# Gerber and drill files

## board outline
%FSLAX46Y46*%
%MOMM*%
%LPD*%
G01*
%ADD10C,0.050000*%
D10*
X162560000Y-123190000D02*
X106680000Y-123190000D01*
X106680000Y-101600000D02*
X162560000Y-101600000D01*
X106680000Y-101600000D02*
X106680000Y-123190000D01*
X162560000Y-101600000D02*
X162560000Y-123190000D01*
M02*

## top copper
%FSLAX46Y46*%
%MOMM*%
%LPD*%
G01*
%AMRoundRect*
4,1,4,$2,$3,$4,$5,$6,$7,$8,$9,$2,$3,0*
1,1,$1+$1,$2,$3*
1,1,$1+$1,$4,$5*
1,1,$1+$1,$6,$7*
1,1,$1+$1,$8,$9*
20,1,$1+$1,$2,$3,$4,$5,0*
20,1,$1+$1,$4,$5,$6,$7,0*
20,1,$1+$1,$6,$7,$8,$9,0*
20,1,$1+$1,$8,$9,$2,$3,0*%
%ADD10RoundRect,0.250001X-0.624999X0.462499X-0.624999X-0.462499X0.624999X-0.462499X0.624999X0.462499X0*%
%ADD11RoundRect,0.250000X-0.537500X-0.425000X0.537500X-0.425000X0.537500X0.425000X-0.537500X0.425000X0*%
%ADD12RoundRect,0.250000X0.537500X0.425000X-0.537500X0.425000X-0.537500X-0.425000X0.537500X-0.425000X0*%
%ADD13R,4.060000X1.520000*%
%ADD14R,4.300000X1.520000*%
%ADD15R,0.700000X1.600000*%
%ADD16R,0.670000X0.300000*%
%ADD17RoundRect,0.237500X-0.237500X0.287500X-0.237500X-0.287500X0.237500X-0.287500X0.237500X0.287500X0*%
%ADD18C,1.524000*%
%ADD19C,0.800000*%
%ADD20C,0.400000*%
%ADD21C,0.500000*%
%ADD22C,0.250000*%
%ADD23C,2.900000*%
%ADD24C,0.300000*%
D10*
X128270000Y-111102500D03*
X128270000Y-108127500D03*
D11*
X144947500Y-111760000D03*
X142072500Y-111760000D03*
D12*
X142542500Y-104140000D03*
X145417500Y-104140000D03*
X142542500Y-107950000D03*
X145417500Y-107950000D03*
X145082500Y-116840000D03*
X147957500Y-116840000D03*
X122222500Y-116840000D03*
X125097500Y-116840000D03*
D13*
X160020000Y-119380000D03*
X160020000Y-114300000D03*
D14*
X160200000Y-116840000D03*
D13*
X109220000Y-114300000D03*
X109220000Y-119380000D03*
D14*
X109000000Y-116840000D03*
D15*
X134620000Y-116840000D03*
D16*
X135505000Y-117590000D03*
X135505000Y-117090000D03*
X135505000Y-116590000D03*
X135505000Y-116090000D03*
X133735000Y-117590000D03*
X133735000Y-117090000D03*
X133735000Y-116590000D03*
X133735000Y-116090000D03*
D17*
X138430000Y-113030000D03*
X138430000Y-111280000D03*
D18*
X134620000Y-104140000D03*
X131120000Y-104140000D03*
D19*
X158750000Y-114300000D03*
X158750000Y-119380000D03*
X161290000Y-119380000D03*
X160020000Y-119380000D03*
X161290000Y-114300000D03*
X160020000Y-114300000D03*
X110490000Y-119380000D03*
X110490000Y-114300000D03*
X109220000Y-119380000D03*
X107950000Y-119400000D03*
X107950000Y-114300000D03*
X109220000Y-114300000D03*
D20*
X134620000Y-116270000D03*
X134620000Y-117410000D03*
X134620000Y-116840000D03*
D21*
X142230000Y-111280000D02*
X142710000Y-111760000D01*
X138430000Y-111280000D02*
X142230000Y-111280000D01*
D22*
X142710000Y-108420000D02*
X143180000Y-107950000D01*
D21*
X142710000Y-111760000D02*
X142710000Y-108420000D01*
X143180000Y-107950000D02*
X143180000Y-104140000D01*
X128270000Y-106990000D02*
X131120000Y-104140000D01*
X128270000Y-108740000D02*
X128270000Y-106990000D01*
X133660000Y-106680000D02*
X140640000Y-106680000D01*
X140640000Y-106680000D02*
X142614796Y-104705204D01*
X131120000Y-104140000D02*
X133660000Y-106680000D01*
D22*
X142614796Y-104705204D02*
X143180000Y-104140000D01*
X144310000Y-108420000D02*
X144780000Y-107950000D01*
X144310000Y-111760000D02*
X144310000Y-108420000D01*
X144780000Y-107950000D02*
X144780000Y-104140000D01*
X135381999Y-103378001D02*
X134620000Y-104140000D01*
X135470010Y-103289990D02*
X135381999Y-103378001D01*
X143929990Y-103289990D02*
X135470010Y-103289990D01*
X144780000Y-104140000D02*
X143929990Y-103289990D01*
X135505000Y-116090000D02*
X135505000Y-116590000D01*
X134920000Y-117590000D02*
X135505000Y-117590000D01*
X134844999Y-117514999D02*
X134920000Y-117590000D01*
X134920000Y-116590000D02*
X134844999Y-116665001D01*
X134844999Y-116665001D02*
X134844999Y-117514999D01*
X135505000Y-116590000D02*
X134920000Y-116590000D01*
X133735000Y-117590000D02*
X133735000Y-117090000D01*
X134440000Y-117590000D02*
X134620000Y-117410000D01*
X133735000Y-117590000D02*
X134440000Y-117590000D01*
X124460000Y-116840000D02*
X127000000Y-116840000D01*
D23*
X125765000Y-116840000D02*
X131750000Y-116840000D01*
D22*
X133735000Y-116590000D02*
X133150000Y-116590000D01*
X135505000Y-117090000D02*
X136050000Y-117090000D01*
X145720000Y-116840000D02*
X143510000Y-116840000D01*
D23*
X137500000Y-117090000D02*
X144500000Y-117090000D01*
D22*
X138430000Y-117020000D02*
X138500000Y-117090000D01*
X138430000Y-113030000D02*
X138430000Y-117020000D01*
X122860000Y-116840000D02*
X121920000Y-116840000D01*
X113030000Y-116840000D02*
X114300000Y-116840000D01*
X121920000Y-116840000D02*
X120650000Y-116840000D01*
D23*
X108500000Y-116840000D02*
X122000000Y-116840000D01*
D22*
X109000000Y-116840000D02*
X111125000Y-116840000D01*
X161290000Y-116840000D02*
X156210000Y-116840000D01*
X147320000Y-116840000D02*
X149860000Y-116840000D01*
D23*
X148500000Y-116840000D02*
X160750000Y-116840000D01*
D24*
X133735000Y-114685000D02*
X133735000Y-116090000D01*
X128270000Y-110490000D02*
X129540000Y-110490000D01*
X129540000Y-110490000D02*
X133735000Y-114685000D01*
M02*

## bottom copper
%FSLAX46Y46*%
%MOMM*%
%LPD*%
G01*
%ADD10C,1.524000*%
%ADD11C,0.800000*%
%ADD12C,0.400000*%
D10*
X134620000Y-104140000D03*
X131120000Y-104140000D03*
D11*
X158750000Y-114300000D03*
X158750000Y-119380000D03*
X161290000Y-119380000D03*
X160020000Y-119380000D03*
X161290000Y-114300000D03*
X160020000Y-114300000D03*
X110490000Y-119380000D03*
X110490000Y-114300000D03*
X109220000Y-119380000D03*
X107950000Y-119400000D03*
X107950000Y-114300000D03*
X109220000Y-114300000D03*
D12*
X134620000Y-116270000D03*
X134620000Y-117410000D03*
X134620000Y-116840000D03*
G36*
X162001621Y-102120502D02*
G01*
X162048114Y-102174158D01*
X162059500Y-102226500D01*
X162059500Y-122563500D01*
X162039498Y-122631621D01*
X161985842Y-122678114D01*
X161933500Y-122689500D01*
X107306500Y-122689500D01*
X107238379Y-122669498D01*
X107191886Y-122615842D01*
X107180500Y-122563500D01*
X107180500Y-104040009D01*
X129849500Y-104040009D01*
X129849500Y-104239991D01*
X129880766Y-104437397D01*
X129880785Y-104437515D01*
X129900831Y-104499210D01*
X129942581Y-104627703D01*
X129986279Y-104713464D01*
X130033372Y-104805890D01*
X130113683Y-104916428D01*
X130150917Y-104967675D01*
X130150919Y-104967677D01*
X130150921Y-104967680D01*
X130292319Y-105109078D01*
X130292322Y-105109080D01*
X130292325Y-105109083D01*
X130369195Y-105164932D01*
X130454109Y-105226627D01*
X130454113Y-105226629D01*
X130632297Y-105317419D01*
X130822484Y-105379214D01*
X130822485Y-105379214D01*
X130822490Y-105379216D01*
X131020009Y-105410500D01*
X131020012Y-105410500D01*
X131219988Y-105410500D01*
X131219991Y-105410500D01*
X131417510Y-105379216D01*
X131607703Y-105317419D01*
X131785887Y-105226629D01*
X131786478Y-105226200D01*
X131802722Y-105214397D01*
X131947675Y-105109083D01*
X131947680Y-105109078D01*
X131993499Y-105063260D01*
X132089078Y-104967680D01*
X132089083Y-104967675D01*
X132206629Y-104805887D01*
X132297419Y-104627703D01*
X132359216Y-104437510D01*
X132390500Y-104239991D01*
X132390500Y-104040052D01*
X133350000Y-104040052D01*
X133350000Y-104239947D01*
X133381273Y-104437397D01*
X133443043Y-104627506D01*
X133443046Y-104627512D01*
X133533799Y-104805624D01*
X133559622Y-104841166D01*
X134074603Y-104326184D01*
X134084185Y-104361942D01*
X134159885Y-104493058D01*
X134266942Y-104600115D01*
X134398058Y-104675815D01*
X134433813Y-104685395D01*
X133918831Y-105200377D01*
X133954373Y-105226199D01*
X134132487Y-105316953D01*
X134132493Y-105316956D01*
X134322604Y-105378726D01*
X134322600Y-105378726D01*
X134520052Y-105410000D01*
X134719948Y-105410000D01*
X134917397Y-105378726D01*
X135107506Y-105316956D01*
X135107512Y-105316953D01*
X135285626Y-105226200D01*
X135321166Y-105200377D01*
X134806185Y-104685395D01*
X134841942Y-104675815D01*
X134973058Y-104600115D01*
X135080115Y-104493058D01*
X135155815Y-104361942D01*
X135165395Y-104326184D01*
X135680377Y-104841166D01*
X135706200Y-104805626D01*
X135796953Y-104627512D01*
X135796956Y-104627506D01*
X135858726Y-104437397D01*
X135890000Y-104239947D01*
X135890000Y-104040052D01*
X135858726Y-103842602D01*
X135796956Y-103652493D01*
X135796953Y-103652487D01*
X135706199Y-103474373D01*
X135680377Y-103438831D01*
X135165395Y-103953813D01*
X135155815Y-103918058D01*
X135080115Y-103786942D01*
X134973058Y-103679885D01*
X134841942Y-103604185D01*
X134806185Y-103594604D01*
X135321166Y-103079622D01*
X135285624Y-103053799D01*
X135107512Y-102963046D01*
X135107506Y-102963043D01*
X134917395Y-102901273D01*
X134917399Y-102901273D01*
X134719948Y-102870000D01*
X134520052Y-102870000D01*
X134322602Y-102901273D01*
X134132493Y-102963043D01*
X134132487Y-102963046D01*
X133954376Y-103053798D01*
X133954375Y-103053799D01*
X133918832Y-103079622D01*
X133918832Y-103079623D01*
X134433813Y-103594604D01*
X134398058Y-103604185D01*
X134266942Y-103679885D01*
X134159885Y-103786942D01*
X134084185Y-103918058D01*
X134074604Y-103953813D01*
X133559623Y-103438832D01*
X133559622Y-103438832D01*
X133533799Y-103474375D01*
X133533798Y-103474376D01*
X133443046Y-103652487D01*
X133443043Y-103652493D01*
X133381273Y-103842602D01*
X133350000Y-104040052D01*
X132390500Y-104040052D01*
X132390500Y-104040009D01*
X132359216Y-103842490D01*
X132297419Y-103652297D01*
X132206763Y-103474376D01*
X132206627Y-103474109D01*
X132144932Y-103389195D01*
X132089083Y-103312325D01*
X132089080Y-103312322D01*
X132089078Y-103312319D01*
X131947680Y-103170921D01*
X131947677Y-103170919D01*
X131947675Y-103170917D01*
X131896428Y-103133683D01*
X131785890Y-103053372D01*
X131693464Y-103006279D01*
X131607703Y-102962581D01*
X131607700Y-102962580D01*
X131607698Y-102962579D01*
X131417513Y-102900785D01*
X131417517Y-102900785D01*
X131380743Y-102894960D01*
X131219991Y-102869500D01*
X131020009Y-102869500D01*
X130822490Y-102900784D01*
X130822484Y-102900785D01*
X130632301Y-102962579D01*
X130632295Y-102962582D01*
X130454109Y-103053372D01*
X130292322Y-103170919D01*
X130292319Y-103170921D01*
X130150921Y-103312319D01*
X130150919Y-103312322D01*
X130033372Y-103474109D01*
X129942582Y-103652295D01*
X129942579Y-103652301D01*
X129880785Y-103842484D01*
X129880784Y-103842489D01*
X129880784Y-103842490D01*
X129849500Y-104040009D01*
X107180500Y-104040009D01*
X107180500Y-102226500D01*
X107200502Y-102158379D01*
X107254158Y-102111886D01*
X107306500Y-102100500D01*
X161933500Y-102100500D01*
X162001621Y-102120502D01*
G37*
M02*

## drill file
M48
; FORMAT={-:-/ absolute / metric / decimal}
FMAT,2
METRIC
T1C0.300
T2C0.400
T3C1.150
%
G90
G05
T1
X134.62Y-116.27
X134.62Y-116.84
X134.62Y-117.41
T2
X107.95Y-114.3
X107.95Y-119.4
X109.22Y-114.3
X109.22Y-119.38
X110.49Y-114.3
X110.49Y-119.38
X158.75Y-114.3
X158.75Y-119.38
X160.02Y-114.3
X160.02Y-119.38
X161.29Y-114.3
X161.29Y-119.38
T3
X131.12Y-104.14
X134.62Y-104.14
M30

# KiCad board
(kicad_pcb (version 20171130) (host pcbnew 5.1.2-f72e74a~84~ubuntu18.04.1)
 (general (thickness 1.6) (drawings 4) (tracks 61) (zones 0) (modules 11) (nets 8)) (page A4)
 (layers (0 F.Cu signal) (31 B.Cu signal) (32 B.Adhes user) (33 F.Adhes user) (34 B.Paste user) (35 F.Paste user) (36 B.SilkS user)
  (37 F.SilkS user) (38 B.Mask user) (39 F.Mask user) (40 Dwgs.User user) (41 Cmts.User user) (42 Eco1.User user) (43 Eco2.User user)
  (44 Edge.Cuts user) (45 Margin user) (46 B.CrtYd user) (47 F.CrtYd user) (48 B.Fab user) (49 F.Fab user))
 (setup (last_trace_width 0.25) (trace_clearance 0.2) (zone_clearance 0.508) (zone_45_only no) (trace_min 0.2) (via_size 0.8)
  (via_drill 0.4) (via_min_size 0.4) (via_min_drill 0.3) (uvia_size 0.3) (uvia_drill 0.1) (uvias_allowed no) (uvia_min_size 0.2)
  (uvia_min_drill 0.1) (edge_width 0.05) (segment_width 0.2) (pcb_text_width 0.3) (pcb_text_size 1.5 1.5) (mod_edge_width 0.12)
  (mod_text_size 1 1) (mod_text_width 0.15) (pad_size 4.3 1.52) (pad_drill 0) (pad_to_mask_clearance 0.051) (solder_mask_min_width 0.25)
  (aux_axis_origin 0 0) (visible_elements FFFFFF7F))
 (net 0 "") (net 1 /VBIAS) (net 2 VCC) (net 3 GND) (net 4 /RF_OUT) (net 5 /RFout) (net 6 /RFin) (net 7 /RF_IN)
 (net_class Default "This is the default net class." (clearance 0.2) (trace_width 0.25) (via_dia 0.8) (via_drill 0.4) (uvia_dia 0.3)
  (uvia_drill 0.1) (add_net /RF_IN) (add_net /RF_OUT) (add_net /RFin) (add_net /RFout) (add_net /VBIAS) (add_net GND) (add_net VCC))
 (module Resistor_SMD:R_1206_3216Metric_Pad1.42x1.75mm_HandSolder (layer F.Cu) (at 128.27 109.615 270)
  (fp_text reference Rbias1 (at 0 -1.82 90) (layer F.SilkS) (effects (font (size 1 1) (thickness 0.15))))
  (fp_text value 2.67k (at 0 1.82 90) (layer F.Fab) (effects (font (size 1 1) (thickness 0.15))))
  (pad 2 smd roundrect (at 1.4875 0 270) (size 1.425 1.75) (layers F.Cu F.Paste F.Mask) (roundrect_rratio 0.175439) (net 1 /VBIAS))
  (pad 1 smd roundrect (at -1.4875 0 270) (size 1.425 1.75) (layers F.Cu F.Paste F.Mask) (roundrect_rratio 0.175439) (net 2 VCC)))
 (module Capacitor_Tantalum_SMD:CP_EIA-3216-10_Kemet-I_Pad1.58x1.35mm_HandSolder (layer F.Cu) (at 143.51 111.76)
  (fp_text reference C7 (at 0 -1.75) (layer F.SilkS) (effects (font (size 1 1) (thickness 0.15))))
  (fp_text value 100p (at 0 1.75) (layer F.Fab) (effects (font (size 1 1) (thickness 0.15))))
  (pad 2 smd roundrect (at 1.4375 0) (size 1.575 1.35) (layers F.Cu F.Paste F.Mask) (roundrect_rratio 0.185185) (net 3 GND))
  (pad 1 smd roundrect (at -1.4375 0) (size 1.575 1.35) (layers F.Cu F.Paste F.Mask) (roundrect_rratio 0.185185) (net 2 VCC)))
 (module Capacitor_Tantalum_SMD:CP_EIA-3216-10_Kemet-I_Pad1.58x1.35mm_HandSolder (layer F.Cu) (at 143.98 104.14 180)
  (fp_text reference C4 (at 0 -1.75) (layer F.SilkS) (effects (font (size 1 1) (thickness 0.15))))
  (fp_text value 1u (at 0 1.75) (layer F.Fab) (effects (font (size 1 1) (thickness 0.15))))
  (pad 2 smd roundrect (at 1.4375 0 180) (size 1.575 1.35) (layers F.Cu F.Paste F.Mask) (roundrect_rratio 0.185185) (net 2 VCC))
  (pad 1 smd roundrect (at -1.4375 0 180) (size 1.575 1.35) (layers F.Cu F.Paste F.Mask) (roundrect_rratio 0.185185) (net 3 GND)))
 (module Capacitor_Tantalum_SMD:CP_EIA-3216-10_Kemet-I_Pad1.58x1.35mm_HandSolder (layer F.Cu) (at 143.98 107.95 180)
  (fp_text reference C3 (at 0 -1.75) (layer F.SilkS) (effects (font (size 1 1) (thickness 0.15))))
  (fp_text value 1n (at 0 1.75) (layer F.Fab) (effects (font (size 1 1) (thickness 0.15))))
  (pad 2 smd roundrect (at 1.4375 0 180) (size 1.575 1.35) (layers F.Cu F.Paste F.Mask) (roundrect_rratio 0.185185) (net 2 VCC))
  (pad 1 smd roundrect (at -1.4375 0 180) (size 1.575 1.35) (layers F.Cu F.Paste F.Mask) (roundrect_rratio 0.185185) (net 3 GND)))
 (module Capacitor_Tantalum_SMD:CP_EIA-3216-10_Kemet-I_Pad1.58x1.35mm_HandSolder (layer F.Cu) (at 146.52 116.84 180)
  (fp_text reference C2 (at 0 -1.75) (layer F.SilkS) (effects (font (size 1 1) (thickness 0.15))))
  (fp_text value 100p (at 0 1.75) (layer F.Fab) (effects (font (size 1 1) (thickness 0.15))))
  (pad 2 smd roundrect (at 1.4375 0 180) (size 1.575 1.35) (layers F.Cu F.Paste F.Mask) (roundrect_rratio 0.185185) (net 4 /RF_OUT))
  (pad 1 smd roundrect (at -1.4375 0 180) (size 1.575 1.35) (layers F.Cu F.Paste F.Mask) (roundrect_rratio 0.185185) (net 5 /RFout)))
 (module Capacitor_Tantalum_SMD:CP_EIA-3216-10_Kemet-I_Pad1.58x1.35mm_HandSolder (layer F.Cu) (at 123.66 116.84 180)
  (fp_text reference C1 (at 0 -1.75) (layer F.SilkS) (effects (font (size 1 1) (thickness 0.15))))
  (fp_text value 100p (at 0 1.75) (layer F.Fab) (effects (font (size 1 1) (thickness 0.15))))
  (pad 2 smd roundrect (at 1.4375 0 180) (size 1.575 1.35) (layers F.Cu F.Paste F.Mask) (roundrect_rratio 0.185185) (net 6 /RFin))
  (pad 1 smd roundrect (at -1.4375 0 180) (size 1.575 1.35) (layers F.Cu F.Paste F.Mask) (roundrect_rratio 0.185185) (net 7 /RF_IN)))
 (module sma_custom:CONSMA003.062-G (layer F.Cu) (at 163.83 119.38)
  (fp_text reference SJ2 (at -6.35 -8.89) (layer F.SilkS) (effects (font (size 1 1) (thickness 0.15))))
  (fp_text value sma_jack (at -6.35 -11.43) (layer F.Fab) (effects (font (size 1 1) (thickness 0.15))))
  (pad 3 smd rect (at -3.81 0) (size 4.06 1.52) (layers F.Cu F.Paste F.Mask) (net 3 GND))
  (pad 2 smd rect (at -3.81 -5.08) (size 4.06 1.52) (layers F.Cu F.Paste F.Mask) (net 3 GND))
  (pad 1 smd rect (at -3.63 -2.54) (size 4.3 1.52) (layers F.Cu F.Paste F.Mask) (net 5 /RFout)))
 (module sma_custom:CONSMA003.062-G (layer F.Cu) (at 105.41 114.3 180)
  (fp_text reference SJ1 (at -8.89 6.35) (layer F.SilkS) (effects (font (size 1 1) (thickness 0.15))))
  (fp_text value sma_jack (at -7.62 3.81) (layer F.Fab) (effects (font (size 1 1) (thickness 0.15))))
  (pad 3 smd rect (at -3.81 0 180) (size 4.06 1.52) (layers F.Cu F.Paste F.Mask) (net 3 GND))
  (pad 2 smd rect (at -3.81 -5.08 180) (size 4.06 1.52) (layers F.Cu F.Paste F.Mask) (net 3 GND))
  (pad 1 smd rect (at -3.59 -2.54 180) (size 4.3 1.52) (layers F.Cu F.Paste F.Mask) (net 6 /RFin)))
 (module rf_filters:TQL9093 (layer F.Cu) (at 134.62 116.84)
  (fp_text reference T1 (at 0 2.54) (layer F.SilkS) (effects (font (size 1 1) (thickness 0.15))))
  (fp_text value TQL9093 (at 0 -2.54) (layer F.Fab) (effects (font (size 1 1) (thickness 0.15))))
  (pad 9 smd rect (at 0 0) (size 0.7 1.6) (layers F.Cu F.Paste F.Mask) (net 3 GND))
  (pad 8 smd rect (at 0.885 0.75) (size 0.67 0.3) (layers F.Cu F.Paste F.Mask) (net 3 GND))
  (pad 7 smd rect (at 0.885 0.25) (size 0.67 0.3) (layers F.Cu F.Paste F.Mask) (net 4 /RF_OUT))
  (pad 6 smd rect (at 0.885 -0.25) (size 0.67 0.3) (layers F.Cu F.Paste F.Mask) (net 3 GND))
  (pad 5 smd rect (at 0.885 -0.75) (size 0.67 0.3) (layers F.Cu F.Paste F.Mask) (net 3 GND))
  (pad 4 smd rect (at -0.885 0.75) (size 0.67 0.3) (layers F.Cu F.Paste F.Mask) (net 3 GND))
  (pad 3 smd rect (at -0.885 0.25) (size 0.67 0.3) (layers F.Cu F.Paste F.Mask) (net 3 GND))
  (pad 2 smd rect (at -0.885 -0.25) (size 0.67 0.3) (layers F.Cu F.Paste F.Mask) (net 7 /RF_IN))
  (pad 1 smd rect (at -0.885 -0.75) (size 0.67 0.3) (layers F.Cu F.Paste F.Mask) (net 1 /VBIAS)))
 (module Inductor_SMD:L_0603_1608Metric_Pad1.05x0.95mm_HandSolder (layer F.Cu) (at 138.43 112.155 270)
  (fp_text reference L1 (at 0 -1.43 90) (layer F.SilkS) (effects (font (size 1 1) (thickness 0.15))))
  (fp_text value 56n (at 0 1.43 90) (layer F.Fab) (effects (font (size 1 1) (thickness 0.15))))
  (pad 2 smd roundrect (at 0.875 0 270) (size 1.05 0.95) (layers F.Cu F.Paste F.Mask) (roundrect_rratio 0.25) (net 4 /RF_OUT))
  (pad 1 smd roundrect (at -0.875 0 270) (size 1.05 0.95) (layers F.Cu F.Paste F.Mask) (roundrect_rratio 0.25) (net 2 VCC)))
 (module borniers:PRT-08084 (layer F.Cu) (at 134.62 109.22)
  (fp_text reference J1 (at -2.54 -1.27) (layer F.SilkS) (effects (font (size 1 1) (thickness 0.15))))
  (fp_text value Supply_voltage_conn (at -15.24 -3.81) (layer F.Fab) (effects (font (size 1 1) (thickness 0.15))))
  (pad 2 thru_hole circle (at 0 -5.08) (size 1.524 1.524) (drill 1.15) (layers *.Cu *.Mask) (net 3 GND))
  (pad 1 thru_hole circle (at -3.5 -5.08) (size 1.524 1.524) (drill 1.15) (layers *.Cu *.Mask) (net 2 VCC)))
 (gr_line (start 162.56 123.19) (end 106.68 123.19) (layer Edge.Cuts) (width 0.05))
 (gr_line (start 106.68 101.6) (end 162.56 101.6) (layer Edge.Cuts) (width 0.05))
 (gr_line (start 106.68 101.6) (end 106.68 123.19) (layer Edge.Cuts) (width 0.05))
 (gr_line (start 162.56 101.6) (end 162.56 123.19) (layer Edge.Cuts) (width 0.05))
 (segment (start 142.23 111.28) (end 142.71 111.76) (width 0.5) (layer F.Cu) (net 2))
 (segment (start 138.43 111.28) (end 142.23 111.28) (width 0.5) (layer F.Cu) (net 2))
 (segment (start 142.71 108.42) (end 143.18 107.95) (width 0.25) (layer F.Cu) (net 2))
 (segment (start 142.71 111.76) (end 142.71 108.42) (width 0.5) (layer F.Cu) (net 2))
 (segment (start 143.18 107.95) (end 143.18 104.14) (width 0.5) (layer F.Cu) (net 2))
 (segment (start 128.27 106.99) (end 131.12 104.14) (width 0.5) (layer F.Cu) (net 2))
 (segment (start 128.27 108.74) (end 128.27 106.99) (width 0.5) (layer F.Cu) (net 2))
 (segment (start 133.66 106.68) (end 140.64 106.68) (width 0.5) (layer F.Cu) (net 2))
 (segment (start 140.64 106.68) (end 142.614796 104.705204) (width 0.5) (layer F.Cu) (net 2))
 (segment (start 131.12 104.14) (end 133.66 106.68) (width 0.5) (layer F.Cu) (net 2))
 (segment (start 142.614796 104.705204) (end 143.18 104.14) (width 0.25) (layer F.Cu) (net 2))
 (via (at 158.75 114.3) (size 0.8) (drill 0.4) (layers F.Cu B.Cu) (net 3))
 (via (at 158.75 119.38) (size 0.8) (drill 0.4) (layers F.Cu B.Cu) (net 3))
 (via (at 161.29 119.38) (size 0.8) (drill 0.4) (layers F.Cu B.Cu) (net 3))
 (via (at 160.02 119.38) (size 0.8) (drill 0.4) (layers F.Cu B.Cu) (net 3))
 (via (at 161.29 114.3) (size 0.8) (drill 0.4) (layers F.Cu B.Cu) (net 3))
 (via (at 160.02 114.3) (size 0.8) (drill 0.4) (layers F.Cu B.Cu) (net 3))
 (via (at 110.49 119.38) (size 0.8) (drill 0.4) (layers F.Cu B.Cu) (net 3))
 (via (at 110.49 114.3) (size 0.8) (drill 0.4) (layers F.Cu B.Cu) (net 3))
 (via (at 109.22 119.38) (size 0.8) (drill 0.4) (layers F.Cu B.Cu) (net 3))
 (via (at 107.95 119.4) (size 0.8) (drill 0.4) (layers F.Cu B.Cu) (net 3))
 (via (at 107.95 114.3) (size 0.8) (drill 0.4) (layers F.Cu B.Cu) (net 3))
 (via (at 109.22 114.3) (size 0.8) (drill 0.4) (layers F.Cu B.Cu) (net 3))
 (via (at 134.62 116.27) (size 0.4) (drill 0.3) (layers F.Cu B.Cu) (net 3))
 (via (at 134.62 117.41) (size 0.4) (drill 0.3) (layers F.Cu B.Cu) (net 3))
 (via (at 134.62 116.84) (size 0.4) (drill 0.3) (layers F.Cu B.Cu) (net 3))
 (segment (start 144.31 108.42) (end 144.78 107.95) (width 0.25) (layer F.Cu) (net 3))
 (segment (start 144.31 111.76) (end 144.31 108.42) (width 0.25) (layer F.Cu) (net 3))
 (segment (start 144.78 107.95) (end 144.78 104.14) (width 0.25) (layer F.Cu) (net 3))
 (segment (start 135.381999 103.378001) (end 134.62 104.14) (width 0.25) (layer F.Cu) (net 3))
 (segment (start 135.47001 103.28999) (end 135.381999 103.378001) (width 0.25) (layer F.Cu) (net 3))
 (segment (start 143.92999 103.28999) (end 135.47001 103.28999) (width 0.25) (layer F.Cu) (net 3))
 (segment (start 144.78 104.14) (end 143.92999 103.28999) (width 0.25) (layer F.Cu) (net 3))
 (segment (start 135.505 116.09) (end 135.505 116.59) (width 0.25) (layer F.Cu) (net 3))
 (segment (start 134.92 117.59) (end 135.505 117.59) (width 0.25) (layer F.Cu) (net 3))
 (segment (start 134.844999 117.514999) (end 134.92 117.59) (width 0.25) (layer F.Cu) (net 3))
 (segment (start 134.92 116.59) (end 134.844999 116.665001) (width 0.25) (layer F.Cu) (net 3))
 (segment (start 134.844999 116.665001) (end 134.844999 117.514999) (width 0.25) (layer F.Cu) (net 3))
 (segment (start 135.505 116.59) (end 134.92 116.59) (width 0.25) (layer F.Cu) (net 3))
 (segment (start 133.735 117.59) (end 133.735 117.09) (width 0.25) (layer F.Cu) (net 3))
 (segment (start 134.44 117.59) (end 134.62 117.41) (width 0.25) (layer F.Cu) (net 3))
 (segment (start 133.735 117.59) (end 134.44 117.59) (width 0.25) (layer F.Cu) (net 3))
 (segment (start 124.46 116.84) (end 127 116.84) (width 0.25) (layer F.Cu) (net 7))
 (segment (start 125.765 116.84) (end 131.75 116.84) (width 2.9) (layer F.Cu) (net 7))
 (segment (start 133.735 116.59) (end 133.15 116.59) (width 0.25) (layer F.Cu) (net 7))
 (segment (start 135.505 117.09) (end 136.05 117.09) (width 0.25) (layer F.Cu) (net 4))
 (segment (start 145.72 116.84) (end 143.51 116.84) (width 0.25) (layer F.Cu) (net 4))
 (segment (start 137.5 117.09) (end 144.5 117.09) (width 2.9) (layer F.Cu) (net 4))
 (segment (start 138.43 117.02) (end 138.5 117.09) (width 0.25) (layer F.Cu) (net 4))
 (segment (start 138.43 113.03) (end 138.43 117.02) (width 0.25) (layer F.Cu) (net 4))
 (segment (start 122.86 116.84) (end 121.92 116.84) (width 0.25) (layer F.Cu) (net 6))
 (segment (start 113.03 116.84) (end 114.3 116.84) (width 0.25) (layer F.Cu) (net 6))
 (segment (start 121.92 116.84) (end 120.65 116.84) (width 0.25) (layer F.Cu) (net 6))
 (segment (start 108.5 116.84) (end 122 116.84) (width 2.9) (layer F.Cu) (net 6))
 (segment (start 109 116.84) (end 111.125 116.84) (width 0.25) (layer F.Cu) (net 6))
 (segment (start 161.29 116.84) (end 156.21 116.84) (width 0.25) (layer F.Cu) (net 5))
 (segment (start 147.32 116.84) (end 149.86 116.84) (width 0.25) (layer F.Cu) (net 5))
 (segment (start 148.5 116.84) (end 160.75 116.84) (width 2.9) (layer F.Cu) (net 5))
 (segment (start 133.735 114.685) (end 133.735 116.09) (width 0.3) (layer F.Cu) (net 1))
 (segment (start 128.27 110.49) (end 129.54 110.49) (width 0.3) (layer F.Cu) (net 1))
 (segment (start 129.54 110.49) (end 133.735 114.685) (width 0.3) (layer F.Cu) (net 1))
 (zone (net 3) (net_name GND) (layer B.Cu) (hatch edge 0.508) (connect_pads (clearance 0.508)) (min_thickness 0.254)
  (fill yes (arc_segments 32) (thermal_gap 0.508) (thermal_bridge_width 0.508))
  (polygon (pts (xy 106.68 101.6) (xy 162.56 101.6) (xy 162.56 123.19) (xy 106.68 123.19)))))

